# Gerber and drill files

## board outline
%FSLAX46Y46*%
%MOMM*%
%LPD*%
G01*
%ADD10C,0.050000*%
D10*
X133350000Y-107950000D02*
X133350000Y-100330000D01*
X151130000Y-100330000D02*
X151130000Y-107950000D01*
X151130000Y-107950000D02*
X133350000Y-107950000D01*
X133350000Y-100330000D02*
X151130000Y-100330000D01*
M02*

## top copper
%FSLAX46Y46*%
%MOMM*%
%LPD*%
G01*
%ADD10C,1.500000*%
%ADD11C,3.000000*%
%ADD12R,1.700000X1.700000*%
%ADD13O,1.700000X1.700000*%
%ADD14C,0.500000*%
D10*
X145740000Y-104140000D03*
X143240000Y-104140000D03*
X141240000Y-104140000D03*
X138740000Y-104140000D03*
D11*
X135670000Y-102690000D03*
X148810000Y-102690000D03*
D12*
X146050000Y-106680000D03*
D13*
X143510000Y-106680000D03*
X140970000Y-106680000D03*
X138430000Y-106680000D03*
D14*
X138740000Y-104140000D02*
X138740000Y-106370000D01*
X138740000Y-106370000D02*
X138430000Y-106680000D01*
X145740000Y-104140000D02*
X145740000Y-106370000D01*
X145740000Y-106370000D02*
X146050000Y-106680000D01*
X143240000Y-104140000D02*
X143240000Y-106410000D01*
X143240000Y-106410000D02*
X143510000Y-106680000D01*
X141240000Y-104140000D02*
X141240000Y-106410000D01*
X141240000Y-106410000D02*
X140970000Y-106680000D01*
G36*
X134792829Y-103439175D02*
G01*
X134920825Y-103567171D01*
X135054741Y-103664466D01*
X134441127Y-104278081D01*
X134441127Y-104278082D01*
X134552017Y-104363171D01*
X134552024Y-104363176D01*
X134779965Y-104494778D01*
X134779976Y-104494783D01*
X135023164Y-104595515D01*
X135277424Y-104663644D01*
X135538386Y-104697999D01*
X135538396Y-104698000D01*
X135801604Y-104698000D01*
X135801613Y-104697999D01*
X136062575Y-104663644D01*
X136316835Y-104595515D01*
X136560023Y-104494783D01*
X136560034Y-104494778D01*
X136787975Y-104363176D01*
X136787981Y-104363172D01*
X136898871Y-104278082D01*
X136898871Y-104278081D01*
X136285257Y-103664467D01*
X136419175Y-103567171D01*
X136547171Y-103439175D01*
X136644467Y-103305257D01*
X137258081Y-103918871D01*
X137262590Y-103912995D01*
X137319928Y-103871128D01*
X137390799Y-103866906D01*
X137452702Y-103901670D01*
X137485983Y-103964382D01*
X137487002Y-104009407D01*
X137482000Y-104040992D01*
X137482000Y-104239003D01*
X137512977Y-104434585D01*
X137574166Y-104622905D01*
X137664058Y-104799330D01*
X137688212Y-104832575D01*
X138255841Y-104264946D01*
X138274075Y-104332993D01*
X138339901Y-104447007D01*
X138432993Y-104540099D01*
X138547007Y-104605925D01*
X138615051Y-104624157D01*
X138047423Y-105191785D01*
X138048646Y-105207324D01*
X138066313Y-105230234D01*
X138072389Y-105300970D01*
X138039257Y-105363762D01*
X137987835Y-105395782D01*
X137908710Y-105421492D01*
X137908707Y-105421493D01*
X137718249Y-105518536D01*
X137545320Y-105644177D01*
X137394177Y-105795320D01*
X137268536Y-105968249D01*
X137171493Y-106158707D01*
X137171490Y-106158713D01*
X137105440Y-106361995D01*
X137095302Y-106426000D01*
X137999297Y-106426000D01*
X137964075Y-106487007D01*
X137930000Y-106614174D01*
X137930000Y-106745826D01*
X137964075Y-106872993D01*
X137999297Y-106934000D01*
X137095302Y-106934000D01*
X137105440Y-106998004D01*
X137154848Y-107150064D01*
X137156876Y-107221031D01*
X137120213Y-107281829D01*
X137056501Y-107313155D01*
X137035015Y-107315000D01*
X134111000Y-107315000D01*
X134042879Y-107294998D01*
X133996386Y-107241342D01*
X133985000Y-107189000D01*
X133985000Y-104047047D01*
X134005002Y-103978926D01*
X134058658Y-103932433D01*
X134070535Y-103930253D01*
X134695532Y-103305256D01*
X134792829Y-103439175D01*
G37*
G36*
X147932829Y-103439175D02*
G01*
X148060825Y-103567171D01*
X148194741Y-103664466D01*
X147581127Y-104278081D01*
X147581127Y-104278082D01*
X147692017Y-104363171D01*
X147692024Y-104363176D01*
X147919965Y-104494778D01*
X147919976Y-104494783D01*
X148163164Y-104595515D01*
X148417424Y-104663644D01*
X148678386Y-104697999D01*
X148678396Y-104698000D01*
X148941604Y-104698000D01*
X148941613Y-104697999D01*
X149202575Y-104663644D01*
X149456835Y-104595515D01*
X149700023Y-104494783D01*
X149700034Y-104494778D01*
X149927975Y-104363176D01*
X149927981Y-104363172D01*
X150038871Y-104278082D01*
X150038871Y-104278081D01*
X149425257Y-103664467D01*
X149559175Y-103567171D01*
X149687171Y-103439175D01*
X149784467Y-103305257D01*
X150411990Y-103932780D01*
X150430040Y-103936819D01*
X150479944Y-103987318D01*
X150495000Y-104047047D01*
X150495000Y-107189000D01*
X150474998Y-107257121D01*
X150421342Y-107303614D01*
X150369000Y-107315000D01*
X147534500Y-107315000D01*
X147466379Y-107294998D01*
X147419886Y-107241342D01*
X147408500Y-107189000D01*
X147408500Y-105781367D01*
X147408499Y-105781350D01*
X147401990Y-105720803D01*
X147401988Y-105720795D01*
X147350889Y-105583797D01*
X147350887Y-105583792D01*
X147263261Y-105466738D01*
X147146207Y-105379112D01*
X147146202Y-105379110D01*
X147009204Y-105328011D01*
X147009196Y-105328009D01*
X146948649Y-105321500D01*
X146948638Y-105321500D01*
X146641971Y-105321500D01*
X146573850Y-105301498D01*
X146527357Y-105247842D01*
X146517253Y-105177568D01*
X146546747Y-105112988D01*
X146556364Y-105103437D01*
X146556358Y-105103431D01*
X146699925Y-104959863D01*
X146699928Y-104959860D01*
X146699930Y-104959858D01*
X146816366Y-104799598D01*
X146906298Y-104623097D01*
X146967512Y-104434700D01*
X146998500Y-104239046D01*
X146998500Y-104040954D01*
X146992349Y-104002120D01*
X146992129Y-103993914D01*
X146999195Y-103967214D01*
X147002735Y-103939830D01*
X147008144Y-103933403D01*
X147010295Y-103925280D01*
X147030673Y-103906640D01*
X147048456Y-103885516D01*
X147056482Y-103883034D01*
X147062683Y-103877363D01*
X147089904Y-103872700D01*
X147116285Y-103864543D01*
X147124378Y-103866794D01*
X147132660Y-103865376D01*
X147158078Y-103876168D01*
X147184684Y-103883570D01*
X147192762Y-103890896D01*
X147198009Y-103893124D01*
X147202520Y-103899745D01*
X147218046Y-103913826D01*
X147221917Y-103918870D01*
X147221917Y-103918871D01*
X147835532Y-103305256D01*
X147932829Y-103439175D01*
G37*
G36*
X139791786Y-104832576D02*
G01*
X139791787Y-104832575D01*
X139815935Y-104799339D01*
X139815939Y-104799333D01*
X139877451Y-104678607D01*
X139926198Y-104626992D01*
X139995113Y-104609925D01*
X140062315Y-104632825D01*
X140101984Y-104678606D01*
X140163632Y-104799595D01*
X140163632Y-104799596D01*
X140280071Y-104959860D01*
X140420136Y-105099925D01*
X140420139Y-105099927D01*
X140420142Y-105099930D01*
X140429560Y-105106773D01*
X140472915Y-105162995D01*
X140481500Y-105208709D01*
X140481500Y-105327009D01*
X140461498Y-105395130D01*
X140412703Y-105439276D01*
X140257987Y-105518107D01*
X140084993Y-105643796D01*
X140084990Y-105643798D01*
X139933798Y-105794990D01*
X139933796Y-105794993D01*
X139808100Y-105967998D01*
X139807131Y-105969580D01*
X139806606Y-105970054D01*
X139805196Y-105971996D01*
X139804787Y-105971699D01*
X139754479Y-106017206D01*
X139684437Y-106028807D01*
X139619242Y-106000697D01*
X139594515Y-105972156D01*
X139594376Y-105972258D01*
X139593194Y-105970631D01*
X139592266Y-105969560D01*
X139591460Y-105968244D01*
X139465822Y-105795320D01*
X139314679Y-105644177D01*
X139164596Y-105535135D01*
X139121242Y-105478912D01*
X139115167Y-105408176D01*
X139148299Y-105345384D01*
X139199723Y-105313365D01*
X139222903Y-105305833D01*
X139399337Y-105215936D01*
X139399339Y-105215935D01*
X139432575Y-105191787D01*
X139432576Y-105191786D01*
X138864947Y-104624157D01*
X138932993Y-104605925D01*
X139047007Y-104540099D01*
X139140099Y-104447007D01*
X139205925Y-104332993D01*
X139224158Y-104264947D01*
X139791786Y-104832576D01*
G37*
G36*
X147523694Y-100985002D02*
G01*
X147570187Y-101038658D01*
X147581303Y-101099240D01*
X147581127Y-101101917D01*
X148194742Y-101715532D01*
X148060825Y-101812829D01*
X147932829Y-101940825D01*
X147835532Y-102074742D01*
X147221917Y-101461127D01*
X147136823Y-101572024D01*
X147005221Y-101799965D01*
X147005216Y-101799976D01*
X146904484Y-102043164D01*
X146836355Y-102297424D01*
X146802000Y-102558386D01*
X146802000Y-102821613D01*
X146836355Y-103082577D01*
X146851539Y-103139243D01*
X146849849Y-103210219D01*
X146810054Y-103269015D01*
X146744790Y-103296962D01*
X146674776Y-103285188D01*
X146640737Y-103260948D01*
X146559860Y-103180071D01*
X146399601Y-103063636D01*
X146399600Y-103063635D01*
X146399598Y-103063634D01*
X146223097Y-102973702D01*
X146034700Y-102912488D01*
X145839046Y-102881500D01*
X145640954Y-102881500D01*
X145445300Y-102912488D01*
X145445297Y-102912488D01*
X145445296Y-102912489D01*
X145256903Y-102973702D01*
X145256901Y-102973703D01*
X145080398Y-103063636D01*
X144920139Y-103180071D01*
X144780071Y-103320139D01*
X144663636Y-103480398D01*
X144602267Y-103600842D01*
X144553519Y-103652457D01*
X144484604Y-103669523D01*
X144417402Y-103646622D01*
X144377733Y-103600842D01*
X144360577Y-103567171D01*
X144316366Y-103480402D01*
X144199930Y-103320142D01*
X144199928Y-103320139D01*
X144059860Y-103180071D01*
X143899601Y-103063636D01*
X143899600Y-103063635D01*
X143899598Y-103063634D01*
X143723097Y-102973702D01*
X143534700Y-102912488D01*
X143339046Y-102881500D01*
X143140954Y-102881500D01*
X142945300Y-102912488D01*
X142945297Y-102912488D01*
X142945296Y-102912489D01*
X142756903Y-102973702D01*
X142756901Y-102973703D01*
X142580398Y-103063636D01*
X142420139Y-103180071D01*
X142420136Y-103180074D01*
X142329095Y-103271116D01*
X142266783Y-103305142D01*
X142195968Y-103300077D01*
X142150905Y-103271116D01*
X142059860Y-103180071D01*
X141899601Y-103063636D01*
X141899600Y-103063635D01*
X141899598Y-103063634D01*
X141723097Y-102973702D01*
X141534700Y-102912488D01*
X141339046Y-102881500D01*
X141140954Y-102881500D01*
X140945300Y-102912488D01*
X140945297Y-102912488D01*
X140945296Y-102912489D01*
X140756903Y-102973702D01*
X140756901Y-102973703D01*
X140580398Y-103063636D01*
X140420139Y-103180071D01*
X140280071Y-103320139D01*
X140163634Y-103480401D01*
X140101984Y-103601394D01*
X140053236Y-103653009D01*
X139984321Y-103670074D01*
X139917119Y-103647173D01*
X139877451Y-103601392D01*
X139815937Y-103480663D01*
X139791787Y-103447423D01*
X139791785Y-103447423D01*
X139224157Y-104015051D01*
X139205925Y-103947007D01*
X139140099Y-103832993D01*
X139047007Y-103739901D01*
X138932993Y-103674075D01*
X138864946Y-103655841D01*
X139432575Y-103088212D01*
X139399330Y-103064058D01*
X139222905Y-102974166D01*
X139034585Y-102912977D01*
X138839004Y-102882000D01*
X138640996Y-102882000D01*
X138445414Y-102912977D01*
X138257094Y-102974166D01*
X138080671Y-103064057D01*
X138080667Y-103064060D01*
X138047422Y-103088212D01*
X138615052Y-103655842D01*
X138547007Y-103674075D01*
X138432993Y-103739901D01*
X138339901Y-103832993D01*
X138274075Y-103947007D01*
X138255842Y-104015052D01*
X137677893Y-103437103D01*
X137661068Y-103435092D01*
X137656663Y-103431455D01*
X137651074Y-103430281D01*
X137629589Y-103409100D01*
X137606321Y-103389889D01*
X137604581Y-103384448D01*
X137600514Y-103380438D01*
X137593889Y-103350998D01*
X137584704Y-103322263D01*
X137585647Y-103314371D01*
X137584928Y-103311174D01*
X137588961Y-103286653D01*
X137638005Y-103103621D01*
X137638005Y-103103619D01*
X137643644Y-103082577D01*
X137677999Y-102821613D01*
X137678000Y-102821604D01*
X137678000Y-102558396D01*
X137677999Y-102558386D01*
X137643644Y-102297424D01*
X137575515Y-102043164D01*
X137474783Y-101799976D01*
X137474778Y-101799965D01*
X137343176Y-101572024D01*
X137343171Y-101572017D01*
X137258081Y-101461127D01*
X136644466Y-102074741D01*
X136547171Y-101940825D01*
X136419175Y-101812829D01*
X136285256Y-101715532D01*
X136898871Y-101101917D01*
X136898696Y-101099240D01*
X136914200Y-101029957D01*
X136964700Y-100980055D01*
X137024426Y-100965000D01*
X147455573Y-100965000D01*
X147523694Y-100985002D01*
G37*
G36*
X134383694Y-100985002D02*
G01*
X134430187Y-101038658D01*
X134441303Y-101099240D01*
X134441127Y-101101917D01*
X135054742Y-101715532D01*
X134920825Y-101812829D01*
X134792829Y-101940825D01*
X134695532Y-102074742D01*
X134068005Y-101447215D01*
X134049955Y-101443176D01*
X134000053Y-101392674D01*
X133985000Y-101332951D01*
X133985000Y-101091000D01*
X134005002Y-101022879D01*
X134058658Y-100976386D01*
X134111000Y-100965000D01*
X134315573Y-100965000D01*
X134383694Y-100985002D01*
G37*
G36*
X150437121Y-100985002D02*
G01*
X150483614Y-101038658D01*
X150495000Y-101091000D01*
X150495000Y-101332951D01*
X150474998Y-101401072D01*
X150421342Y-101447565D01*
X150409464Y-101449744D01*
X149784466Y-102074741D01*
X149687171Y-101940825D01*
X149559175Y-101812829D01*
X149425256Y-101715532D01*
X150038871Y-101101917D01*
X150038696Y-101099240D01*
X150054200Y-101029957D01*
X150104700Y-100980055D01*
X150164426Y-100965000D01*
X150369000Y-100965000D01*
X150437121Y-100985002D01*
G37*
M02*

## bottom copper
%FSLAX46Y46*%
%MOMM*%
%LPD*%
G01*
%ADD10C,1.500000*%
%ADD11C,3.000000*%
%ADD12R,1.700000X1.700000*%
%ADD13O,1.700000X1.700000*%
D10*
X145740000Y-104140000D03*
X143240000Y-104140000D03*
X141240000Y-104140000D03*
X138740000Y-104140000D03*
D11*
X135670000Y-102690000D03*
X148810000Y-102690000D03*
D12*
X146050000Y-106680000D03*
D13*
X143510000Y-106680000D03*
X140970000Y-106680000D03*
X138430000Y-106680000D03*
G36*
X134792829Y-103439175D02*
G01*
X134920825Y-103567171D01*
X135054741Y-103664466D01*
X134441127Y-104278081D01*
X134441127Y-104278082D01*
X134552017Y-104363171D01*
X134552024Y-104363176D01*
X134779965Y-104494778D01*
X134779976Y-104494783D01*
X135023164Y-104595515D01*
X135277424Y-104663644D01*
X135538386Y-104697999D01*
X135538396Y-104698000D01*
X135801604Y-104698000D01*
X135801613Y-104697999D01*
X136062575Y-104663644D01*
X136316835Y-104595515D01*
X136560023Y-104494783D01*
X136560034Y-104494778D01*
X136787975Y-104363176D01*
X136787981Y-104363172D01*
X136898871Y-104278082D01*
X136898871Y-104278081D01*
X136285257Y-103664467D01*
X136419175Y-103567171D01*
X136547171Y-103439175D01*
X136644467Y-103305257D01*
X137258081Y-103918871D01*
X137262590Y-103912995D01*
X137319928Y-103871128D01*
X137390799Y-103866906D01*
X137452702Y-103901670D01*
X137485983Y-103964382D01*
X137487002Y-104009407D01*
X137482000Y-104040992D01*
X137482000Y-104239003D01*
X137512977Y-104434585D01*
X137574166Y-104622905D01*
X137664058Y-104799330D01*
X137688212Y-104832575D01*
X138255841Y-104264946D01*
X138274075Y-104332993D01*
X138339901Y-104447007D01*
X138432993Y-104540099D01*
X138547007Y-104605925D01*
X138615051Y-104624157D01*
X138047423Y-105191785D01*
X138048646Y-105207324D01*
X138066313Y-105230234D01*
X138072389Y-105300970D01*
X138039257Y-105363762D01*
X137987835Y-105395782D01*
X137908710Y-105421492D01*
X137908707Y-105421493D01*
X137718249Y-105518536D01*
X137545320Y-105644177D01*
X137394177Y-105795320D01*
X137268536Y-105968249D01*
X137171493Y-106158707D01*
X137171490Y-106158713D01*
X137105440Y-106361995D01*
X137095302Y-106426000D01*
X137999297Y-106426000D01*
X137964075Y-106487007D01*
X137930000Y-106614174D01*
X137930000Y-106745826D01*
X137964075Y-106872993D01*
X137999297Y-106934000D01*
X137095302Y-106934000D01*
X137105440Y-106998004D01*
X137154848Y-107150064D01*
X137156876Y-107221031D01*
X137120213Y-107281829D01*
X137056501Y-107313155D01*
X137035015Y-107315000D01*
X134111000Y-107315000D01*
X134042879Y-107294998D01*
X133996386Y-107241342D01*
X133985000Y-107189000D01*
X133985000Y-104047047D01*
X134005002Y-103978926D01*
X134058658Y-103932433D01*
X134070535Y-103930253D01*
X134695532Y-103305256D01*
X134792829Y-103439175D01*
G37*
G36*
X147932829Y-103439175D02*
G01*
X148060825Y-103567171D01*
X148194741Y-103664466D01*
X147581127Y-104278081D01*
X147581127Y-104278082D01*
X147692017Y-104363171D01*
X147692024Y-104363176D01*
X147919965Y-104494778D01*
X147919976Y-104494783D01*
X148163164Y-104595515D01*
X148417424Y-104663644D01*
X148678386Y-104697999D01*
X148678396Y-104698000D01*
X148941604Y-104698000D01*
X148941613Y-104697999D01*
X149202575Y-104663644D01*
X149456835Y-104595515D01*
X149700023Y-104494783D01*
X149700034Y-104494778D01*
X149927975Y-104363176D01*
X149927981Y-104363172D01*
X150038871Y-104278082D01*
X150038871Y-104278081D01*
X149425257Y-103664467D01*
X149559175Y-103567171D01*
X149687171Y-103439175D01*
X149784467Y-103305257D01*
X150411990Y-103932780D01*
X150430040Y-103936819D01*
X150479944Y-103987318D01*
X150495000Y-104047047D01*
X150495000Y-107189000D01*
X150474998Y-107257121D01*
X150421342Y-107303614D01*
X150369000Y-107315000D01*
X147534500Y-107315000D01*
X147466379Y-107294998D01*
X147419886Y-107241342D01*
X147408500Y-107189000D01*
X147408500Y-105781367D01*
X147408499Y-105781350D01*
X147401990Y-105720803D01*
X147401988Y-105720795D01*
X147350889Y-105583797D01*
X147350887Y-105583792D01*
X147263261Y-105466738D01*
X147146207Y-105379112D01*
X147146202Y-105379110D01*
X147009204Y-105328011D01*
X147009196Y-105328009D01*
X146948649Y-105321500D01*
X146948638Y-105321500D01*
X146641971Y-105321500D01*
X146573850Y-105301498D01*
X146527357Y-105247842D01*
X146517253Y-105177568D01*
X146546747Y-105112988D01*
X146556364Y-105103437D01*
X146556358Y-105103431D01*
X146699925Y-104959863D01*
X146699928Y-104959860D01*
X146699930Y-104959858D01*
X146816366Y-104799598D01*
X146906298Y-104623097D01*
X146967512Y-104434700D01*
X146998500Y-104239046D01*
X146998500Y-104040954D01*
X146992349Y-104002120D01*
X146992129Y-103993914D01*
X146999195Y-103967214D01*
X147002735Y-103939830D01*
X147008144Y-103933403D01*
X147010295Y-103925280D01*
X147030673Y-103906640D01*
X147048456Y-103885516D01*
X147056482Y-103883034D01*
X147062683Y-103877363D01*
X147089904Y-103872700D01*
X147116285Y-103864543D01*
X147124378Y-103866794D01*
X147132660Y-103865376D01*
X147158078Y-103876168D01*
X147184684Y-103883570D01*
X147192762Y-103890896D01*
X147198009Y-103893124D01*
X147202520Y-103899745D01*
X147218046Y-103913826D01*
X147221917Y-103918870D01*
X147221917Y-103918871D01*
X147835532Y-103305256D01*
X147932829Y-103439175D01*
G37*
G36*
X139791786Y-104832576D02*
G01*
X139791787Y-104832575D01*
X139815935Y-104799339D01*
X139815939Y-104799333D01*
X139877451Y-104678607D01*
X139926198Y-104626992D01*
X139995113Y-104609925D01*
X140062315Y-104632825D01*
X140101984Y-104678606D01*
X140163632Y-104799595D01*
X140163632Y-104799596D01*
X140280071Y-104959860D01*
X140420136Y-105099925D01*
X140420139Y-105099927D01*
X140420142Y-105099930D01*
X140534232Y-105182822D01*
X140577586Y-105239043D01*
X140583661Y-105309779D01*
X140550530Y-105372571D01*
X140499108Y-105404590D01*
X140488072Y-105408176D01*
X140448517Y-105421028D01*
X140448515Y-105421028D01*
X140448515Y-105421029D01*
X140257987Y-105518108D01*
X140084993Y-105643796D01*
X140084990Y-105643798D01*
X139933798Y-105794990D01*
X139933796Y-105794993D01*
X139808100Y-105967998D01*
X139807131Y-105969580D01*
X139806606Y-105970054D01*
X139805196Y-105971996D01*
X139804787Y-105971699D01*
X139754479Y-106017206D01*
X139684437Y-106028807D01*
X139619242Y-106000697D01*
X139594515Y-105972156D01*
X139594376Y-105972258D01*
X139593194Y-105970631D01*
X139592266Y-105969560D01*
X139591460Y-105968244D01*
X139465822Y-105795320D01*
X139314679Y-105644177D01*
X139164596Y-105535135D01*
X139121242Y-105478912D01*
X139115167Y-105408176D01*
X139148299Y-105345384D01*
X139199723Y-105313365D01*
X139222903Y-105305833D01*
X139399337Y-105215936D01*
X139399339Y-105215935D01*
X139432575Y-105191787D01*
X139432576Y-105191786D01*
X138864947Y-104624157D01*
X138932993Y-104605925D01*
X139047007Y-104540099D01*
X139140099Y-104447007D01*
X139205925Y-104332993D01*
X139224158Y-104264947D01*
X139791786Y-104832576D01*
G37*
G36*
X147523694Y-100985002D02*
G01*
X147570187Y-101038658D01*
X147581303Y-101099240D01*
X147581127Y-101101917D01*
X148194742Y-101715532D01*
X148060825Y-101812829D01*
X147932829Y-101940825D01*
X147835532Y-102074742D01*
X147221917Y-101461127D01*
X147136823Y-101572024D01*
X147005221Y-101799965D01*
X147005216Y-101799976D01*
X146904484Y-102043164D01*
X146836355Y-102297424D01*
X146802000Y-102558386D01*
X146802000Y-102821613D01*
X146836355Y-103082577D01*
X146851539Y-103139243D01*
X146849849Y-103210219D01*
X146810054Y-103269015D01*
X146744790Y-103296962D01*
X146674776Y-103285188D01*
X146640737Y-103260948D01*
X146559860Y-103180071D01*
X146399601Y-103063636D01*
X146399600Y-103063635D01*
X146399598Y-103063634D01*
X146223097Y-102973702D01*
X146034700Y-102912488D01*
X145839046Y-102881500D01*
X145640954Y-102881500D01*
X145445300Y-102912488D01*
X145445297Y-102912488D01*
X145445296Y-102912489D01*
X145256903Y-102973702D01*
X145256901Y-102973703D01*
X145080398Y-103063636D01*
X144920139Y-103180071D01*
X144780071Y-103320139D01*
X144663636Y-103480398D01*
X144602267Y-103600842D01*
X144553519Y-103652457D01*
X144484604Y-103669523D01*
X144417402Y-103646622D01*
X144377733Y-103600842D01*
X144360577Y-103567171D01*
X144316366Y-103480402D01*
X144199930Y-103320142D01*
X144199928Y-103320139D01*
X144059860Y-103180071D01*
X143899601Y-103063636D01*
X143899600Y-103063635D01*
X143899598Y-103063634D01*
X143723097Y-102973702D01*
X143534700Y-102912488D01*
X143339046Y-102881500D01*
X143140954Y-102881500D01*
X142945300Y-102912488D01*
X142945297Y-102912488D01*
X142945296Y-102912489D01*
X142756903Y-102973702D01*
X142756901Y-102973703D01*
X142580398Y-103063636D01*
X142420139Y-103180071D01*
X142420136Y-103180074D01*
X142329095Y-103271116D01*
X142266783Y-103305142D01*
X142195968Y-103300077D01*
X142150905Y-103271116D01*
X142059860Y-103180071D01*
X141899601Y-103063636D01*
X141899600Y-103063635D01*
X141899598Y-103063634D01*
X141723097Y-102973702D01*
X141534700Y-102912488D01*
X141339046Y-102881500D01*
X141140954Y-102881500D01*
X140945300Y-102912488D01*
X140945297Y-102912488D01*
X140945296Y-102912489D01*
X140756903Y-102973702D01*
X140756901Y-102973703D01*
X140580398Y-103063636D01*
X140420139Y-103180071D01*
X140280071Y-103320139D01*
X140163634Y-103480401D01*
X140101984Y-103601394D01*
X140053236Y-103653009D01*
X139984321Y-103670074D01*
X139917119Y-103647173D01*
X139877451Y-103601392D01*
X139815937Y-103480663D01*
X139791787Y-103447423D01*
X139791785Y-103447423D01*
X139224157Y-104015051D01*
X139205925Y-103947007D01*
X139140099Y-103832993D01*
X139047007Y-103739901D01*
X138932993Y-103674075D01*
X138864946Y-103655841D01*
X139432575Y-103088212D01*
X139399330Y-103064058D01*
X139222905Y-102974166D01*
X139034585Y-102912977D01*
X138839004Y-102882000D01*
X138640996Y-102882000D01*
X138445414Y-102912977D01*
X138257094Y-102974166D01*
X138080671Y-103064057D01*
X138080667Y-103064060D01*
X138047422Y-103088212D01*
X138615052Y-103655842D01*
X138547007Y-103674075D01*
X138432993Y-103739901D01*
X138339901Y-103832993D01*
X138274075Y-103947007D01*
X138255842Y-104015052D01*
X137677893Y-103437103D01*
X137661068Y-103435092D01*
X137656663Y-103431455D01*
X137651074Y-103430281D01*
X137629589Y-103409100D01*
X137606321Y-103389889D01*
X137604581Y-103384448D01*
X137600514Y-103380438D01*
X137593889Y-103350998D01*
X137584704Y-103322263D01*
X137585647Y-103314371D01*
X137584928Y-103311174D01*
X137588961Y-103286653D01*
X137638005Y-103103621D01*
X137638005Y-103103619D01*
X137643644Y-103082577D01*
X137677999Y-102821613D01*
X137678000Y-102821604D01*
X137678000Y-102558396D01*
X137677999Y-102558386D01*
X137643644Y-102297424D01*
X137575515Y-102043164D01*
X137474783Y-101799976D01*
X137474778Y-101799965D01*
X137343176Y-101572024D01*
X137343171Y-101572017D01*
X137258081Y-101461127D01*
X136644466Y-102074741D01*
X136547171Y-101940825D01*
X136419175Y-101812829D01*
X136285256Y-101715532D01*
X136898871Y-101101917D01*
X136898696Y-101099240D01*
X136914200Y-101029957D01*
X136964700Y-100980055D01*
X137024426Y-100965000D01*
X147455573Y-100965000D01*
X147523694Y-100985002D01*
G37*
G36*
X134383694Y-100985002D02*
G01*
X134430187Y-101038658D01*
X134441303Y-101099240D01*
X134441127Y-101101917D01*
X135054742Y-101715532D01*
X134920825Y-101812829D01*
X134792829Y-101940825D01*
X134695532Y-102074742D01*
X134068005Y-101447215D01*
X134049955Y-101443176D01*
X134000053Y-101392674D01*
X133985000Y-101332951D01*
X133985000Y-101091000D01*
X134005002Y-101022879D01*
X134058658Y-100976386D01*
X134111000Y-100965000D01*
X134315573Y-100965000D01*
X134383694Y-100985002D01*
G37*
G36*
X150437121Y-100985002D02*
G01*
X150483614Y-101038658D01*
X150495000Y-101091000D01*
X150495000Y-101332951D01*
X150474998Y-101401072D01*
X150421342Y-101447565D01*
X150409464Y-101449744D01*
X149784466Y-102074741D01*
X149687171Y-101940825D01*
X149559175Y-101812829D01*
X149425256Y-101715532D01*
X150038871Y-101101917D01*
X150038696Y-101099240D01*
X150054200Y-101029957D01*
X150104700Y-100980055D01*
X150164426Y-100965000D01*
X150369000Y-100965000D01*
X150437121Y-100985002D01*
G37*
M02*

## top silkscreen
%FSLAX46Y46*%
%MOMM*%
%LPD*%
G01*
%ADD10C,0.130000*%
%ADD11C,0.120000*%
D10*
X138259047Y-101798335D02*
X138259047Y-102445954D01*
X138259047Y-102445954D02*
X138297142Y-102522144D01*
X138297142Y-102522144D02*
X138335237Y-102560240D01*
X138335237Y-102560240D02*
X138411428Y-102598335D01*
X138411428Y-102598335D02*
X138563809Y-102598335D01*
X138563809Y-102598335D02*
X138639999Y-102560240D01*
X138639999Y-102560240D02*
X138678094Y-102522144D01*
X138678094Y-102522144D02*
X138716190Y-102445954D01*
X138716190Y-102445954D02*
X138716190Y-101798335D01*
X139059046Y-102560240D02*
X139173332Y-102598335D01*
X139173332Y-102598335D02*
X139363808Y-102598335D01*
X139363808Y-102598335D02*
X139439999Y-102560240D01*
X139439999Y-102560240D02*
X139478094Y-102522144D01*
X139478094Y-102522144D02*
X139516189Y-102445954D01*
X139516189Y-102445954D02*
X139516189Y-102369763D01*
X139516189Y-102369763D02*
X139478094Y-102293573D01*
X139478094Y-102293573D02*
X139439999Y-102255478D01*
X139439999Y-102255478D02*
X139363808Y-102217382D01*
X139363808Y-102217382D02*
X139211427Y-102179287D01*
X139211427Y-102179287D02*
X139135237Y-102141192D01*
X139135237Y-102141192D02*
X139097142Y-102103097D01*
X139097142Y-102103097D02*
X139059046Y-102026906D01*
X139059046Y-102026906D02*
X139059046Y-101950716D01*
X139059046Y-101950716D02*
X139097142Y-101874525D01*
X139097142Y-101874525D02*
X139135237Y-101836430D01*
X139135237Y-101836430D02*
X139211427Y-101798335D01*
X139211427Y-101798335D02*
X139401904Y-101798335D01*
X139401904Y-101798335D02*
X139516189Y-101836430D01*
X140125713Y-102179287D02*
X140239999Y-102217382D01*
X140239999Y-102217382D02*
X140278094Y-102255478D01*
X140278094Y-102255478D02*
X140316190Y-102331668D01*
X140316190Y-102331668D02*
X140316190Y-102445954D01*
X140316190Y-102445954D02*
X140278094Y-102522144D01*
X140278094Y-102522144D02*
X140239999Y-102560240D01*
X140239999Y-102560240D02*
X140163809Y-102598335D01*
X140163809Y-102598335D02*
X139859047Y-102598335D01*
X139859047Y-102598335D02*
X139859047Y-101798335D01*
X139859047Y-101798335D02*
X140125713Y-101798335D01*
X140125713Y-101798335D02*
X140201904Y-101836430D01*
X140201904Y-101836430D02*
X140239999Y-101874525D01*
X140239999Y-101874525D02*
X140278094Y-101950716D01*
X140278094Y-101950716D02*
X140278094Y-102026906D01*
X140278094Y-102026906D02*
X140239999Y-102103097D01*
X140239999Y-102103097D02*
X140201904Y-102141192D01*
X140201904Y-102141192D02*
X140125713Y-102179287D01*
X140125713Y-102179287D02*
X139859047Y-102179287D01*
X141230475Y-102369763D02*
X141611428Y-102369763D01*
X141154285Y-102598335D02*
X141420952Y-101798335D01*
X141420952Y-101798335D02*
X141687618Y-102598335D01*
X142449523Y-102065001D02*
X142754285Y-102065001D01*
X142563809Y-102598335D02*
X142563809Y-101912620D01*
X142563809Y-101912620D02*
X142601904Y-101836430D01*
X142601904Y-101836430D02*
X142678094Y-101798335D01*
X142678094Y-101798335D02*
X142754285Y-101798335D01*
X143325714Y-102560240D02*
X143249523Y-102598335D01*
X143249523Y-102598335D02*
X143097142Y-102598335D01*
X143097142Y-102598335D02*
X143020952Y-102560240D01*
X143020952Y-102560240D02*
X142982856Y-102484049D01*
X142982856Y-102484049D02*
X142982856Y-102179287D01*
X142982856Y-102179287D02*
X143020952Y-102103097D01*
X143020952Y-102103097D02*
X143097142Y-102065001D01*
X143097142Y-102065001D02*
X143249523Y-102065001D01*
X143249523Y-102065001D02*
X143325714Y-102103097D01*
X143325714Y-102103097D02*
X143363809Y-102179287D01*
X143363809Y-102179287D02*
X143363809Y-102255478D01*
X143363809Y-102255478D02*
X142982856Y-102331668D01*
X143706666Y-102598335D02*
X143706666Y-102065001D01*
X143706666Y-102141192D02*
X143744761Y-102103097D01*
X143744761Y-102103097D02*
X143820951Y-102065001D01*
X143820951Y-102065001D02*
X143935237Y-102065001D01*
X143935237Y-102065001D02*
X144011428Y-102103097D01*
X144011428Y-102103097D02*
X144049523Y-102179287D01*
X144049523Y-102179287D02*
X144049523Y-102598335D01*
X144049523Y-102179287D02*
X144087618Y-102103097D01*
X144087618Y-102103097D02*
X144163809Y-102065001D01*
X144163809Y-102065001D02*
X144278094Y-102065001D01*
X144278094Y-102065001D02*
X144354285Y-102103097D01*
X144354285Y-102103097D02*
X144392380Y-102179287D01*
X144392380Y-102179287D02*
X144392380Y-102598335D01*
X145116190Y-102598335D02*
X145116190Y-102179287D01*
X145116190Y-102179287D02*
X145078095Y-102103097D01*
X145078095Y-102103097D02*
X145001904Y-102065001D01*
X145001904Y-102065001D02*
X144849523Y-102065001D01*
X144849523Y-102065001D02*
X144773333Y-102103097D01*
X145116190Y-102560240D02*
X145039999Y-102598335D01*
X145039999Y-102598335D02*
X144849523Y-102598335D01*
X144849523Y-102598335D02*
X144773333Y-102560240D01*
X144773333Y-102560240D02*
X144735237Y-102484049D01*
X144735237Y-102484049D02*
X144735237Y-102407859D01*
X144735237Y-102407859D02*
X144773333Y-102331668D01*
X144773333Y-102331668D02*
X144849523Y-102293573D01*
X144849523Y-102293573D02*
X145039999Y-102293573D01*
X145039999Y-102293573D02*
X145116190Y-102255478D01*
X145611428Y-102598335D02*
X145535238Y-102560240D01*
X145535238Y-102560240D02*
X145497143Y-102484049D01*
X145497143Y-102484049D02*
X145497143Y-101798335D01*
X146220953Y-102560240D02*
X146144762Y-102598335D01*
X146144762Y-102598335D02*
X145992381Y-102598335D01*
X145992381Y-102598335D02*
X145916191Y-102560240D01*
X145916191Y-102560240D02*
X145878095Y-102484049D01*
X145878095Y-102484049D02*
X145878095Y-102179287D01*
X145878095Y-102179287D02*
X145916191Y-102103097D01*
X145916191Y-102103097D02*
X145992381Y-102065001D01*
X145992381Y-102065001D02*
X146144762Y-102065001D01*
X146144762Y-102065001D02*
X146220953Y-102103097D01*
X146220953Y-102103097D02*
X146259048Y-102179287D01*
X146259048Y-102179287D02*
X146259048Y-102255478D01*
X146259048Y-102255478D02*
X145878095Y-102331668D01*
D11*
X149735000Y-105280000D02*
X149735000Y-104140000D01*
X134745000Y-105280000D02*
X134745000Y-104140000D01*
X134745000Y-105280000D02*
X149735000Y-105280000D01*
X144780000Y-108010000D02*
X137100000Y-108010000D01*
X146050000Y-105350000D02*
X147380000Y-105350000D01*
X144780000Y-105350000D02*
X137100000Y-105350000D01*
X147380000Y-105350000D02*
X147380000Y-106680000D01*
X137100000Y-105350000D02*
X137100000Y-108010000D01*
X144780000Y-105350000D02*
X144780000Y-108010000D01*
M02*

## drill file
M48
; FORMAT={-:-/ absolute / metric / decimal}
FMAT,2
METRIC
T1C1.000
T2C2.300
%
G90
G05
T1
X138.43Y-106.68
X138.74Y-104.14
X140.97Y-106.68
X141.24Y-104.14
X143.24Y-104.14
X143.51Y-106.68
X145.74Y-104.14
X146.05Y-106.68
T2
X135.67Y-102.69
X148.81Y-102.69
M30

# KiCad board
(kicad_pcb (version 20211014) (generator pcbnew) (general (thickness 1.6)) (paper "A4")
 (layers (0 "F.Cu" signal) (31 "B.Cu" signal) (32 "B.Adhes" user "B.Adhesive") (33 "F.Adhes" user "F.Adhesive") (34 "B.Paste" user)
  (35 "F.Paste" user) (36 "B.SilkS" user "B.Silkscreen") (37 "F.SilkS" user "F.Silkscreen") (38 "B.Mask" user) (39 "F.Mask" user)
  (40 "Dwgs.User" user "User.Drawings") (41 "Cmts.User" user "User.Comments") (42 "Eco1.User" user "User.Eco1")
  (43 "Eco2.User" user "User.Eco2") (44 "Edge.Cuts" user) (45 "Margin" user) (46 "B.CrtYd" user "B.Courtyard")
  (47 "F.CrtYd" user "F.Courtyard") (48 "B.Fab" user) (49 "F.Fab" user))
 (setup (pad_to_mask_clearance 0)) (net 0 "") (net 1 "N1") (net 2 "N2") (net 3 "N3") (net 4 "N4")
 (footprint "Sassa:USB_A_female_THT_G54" (layer "F.Cu") (at 142.24 104.14 180)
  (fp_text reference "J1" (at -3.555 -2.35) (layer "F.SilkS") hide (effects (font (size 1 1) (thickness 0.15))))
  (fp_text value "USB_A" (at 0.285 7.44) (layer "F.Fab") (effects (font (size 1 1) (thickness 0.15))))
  (fp_line (start -7.495 -1.14) (end -7.495 0) (layer "F.SilkS") (width 0.12))
  (fp_line (start 7.495 -1.14) (end 7.495 0) (layer "F.SilkS") (width 0.12))
  (fp_line (start 7.495 -1.14) (end -7.495 -1.14) (layer "F.SilkS") (width 0.12))
  (pad "1" thru_hole circle locked (at -3.5 0 90) (size 1.5 1.5) (drill 1) (layers *.Cu *.Mask) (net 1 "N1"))
  (pad "2" thru_hole circle locked (at -1 0 90) (size 1.5 1.5) (drill 1) (layers *.Cu *.Mask) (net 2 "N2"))
  (pad "3" thru_hole circle locked (at 1 0 90) (size 1.5 1.5) (drill 1) (layers *.Cu *.Mask) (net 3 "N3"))
  (pad "4" thru_hole circle locked (at 3.5 0 90) (size 1.5 1.5) (drill 1) (layers *.Cu *.Mask) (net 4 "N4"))
  (pad "5" thru_hole circle locked (at 6.57 1.45 90) (size 3 3) (drill 2.3) (layers *.Cu *.Mask) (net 4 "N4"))
  (pad "5" thru_hole circle locked (at -6.57 1.45 90) (size 3 3) (drill 2.3) (layers *.Cu *.Mask) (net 4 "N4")))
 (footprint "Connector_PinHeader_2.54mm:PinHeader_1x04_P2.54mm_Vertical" (layer "F.Cu") (at 146.05 106.68 -90)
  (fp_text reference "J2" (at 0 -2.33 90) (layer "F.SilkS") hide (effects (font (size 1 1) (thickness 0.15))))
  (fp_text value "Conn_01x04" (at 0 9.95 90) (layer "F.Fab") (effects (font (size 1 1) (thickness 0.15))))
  (fp_line (start 1.33 1.27) (end 1.33 8.95) (layer "F.SilkS") (width 0.12))
  (fp_line (start -1.33 0) (end -1.33 -1.33) (layer "F.SilkS") (width 0.12))
  (fp_line (start -1.33 1.27) (end -1.33 8.95) (layer "F.SilkS") (width 0.12))
  (fp_line (start -1.33 -1.33) (end 0 -1.33) (layer "F.SilkS") (width 0.12))
  (fp_line (start -1.33 8.95) (end 1.33 8.95) (layer "F.SilkS") (width 0.12))
  (fp_line (start -1.33 1.27) (end 1.33 1.27) (layer "F.SilkS") (width 0.12))
  (pad "1" thru_hole rect (at 0 0 270) (size 1.7 1.7) (drill 1) (layers *.Cu *.Mask) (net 1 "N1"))
  (pad "2" thru_hole oval (at 0 2.54 270) (size 1.7 1.7) (drill 1) (layers *.Cu *.Mask) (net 2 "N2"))
  (pad "3" thru_hole oval (at 0 5.08 270) (size 1.7 1.7) (drill 1) (layers *.Cu *.Mask) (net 3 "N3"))
  (pad "4" thru_hole oval (at 0 7.62 270) (size 1.7 1.7) (drill 1) (layers *.Cu *.Mask) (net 4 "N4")))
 (gr_line (start 133.35 107.95) (end 133.35 100.33) (layer "Edge.Cuts") (width 0.05))
 (gr_line (start 151.13 100.33) (end 151.13 107.95) (layer "Edge.Cuts") (width 0.05))
 (gr_line (start 151.13 107.95) (end 133.35 107.95) (layer "Edge.Cuts") (width 0.05))
 (gr_line (start 133.35 100.33) (end 151.13 100.33) (layer "Edge.Cuts") (width 0.05))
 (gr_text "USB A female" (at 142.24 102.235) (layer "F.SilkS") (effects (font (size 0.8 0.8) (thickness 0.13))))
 (segment (start 138.74 104.14) (end 138.74 106.37) (width 0.5) (layer "F.Cu") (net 4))
 (segment (start 138.74 106.37) (end 138.43 106.68) (width 0.5) (layer "F.Cu") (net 4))
 (segment (start 145.74 104.14) (end 145.74 106.37) (width 0.5) (layer "F.Cu") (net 1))
 (segment (start 145.74 106.37) (end 146.05 106.68) (width 0.5) (layer "F.Cu") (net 1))
 (segment (start 143.24 104.14) (end 143.24 106.41) (width 0.5) (layer "F.Cu") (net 2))
 (segment (start 143.24 106.41) (end 143.51 106.68) (width 0.5) (layer "F.Cu") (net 2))
 (segment (start 141.24 104.14) (end 141.24 106.41) (width 0.5) (layer "F.Cu") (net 3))
 (segment (start 141.24 106.41) (end 140.97 106.68) (width 0.5) (layer "F.Cu") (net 3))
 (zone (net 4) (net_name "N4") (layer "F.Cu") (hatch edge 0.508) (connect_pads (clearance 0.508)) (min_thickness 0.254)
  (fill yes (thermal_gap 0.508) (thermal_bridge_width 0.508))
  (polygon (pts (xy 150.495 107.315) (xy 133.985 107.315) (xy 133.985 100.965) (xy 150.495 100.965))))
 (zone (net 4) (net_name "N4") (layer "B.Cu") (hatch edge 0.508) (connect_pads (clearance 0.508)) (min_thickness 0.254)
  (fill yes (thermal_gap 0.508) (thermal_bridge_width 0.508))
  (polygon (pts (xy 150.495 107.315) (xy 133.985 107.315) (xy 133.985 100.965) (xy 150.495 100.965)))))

